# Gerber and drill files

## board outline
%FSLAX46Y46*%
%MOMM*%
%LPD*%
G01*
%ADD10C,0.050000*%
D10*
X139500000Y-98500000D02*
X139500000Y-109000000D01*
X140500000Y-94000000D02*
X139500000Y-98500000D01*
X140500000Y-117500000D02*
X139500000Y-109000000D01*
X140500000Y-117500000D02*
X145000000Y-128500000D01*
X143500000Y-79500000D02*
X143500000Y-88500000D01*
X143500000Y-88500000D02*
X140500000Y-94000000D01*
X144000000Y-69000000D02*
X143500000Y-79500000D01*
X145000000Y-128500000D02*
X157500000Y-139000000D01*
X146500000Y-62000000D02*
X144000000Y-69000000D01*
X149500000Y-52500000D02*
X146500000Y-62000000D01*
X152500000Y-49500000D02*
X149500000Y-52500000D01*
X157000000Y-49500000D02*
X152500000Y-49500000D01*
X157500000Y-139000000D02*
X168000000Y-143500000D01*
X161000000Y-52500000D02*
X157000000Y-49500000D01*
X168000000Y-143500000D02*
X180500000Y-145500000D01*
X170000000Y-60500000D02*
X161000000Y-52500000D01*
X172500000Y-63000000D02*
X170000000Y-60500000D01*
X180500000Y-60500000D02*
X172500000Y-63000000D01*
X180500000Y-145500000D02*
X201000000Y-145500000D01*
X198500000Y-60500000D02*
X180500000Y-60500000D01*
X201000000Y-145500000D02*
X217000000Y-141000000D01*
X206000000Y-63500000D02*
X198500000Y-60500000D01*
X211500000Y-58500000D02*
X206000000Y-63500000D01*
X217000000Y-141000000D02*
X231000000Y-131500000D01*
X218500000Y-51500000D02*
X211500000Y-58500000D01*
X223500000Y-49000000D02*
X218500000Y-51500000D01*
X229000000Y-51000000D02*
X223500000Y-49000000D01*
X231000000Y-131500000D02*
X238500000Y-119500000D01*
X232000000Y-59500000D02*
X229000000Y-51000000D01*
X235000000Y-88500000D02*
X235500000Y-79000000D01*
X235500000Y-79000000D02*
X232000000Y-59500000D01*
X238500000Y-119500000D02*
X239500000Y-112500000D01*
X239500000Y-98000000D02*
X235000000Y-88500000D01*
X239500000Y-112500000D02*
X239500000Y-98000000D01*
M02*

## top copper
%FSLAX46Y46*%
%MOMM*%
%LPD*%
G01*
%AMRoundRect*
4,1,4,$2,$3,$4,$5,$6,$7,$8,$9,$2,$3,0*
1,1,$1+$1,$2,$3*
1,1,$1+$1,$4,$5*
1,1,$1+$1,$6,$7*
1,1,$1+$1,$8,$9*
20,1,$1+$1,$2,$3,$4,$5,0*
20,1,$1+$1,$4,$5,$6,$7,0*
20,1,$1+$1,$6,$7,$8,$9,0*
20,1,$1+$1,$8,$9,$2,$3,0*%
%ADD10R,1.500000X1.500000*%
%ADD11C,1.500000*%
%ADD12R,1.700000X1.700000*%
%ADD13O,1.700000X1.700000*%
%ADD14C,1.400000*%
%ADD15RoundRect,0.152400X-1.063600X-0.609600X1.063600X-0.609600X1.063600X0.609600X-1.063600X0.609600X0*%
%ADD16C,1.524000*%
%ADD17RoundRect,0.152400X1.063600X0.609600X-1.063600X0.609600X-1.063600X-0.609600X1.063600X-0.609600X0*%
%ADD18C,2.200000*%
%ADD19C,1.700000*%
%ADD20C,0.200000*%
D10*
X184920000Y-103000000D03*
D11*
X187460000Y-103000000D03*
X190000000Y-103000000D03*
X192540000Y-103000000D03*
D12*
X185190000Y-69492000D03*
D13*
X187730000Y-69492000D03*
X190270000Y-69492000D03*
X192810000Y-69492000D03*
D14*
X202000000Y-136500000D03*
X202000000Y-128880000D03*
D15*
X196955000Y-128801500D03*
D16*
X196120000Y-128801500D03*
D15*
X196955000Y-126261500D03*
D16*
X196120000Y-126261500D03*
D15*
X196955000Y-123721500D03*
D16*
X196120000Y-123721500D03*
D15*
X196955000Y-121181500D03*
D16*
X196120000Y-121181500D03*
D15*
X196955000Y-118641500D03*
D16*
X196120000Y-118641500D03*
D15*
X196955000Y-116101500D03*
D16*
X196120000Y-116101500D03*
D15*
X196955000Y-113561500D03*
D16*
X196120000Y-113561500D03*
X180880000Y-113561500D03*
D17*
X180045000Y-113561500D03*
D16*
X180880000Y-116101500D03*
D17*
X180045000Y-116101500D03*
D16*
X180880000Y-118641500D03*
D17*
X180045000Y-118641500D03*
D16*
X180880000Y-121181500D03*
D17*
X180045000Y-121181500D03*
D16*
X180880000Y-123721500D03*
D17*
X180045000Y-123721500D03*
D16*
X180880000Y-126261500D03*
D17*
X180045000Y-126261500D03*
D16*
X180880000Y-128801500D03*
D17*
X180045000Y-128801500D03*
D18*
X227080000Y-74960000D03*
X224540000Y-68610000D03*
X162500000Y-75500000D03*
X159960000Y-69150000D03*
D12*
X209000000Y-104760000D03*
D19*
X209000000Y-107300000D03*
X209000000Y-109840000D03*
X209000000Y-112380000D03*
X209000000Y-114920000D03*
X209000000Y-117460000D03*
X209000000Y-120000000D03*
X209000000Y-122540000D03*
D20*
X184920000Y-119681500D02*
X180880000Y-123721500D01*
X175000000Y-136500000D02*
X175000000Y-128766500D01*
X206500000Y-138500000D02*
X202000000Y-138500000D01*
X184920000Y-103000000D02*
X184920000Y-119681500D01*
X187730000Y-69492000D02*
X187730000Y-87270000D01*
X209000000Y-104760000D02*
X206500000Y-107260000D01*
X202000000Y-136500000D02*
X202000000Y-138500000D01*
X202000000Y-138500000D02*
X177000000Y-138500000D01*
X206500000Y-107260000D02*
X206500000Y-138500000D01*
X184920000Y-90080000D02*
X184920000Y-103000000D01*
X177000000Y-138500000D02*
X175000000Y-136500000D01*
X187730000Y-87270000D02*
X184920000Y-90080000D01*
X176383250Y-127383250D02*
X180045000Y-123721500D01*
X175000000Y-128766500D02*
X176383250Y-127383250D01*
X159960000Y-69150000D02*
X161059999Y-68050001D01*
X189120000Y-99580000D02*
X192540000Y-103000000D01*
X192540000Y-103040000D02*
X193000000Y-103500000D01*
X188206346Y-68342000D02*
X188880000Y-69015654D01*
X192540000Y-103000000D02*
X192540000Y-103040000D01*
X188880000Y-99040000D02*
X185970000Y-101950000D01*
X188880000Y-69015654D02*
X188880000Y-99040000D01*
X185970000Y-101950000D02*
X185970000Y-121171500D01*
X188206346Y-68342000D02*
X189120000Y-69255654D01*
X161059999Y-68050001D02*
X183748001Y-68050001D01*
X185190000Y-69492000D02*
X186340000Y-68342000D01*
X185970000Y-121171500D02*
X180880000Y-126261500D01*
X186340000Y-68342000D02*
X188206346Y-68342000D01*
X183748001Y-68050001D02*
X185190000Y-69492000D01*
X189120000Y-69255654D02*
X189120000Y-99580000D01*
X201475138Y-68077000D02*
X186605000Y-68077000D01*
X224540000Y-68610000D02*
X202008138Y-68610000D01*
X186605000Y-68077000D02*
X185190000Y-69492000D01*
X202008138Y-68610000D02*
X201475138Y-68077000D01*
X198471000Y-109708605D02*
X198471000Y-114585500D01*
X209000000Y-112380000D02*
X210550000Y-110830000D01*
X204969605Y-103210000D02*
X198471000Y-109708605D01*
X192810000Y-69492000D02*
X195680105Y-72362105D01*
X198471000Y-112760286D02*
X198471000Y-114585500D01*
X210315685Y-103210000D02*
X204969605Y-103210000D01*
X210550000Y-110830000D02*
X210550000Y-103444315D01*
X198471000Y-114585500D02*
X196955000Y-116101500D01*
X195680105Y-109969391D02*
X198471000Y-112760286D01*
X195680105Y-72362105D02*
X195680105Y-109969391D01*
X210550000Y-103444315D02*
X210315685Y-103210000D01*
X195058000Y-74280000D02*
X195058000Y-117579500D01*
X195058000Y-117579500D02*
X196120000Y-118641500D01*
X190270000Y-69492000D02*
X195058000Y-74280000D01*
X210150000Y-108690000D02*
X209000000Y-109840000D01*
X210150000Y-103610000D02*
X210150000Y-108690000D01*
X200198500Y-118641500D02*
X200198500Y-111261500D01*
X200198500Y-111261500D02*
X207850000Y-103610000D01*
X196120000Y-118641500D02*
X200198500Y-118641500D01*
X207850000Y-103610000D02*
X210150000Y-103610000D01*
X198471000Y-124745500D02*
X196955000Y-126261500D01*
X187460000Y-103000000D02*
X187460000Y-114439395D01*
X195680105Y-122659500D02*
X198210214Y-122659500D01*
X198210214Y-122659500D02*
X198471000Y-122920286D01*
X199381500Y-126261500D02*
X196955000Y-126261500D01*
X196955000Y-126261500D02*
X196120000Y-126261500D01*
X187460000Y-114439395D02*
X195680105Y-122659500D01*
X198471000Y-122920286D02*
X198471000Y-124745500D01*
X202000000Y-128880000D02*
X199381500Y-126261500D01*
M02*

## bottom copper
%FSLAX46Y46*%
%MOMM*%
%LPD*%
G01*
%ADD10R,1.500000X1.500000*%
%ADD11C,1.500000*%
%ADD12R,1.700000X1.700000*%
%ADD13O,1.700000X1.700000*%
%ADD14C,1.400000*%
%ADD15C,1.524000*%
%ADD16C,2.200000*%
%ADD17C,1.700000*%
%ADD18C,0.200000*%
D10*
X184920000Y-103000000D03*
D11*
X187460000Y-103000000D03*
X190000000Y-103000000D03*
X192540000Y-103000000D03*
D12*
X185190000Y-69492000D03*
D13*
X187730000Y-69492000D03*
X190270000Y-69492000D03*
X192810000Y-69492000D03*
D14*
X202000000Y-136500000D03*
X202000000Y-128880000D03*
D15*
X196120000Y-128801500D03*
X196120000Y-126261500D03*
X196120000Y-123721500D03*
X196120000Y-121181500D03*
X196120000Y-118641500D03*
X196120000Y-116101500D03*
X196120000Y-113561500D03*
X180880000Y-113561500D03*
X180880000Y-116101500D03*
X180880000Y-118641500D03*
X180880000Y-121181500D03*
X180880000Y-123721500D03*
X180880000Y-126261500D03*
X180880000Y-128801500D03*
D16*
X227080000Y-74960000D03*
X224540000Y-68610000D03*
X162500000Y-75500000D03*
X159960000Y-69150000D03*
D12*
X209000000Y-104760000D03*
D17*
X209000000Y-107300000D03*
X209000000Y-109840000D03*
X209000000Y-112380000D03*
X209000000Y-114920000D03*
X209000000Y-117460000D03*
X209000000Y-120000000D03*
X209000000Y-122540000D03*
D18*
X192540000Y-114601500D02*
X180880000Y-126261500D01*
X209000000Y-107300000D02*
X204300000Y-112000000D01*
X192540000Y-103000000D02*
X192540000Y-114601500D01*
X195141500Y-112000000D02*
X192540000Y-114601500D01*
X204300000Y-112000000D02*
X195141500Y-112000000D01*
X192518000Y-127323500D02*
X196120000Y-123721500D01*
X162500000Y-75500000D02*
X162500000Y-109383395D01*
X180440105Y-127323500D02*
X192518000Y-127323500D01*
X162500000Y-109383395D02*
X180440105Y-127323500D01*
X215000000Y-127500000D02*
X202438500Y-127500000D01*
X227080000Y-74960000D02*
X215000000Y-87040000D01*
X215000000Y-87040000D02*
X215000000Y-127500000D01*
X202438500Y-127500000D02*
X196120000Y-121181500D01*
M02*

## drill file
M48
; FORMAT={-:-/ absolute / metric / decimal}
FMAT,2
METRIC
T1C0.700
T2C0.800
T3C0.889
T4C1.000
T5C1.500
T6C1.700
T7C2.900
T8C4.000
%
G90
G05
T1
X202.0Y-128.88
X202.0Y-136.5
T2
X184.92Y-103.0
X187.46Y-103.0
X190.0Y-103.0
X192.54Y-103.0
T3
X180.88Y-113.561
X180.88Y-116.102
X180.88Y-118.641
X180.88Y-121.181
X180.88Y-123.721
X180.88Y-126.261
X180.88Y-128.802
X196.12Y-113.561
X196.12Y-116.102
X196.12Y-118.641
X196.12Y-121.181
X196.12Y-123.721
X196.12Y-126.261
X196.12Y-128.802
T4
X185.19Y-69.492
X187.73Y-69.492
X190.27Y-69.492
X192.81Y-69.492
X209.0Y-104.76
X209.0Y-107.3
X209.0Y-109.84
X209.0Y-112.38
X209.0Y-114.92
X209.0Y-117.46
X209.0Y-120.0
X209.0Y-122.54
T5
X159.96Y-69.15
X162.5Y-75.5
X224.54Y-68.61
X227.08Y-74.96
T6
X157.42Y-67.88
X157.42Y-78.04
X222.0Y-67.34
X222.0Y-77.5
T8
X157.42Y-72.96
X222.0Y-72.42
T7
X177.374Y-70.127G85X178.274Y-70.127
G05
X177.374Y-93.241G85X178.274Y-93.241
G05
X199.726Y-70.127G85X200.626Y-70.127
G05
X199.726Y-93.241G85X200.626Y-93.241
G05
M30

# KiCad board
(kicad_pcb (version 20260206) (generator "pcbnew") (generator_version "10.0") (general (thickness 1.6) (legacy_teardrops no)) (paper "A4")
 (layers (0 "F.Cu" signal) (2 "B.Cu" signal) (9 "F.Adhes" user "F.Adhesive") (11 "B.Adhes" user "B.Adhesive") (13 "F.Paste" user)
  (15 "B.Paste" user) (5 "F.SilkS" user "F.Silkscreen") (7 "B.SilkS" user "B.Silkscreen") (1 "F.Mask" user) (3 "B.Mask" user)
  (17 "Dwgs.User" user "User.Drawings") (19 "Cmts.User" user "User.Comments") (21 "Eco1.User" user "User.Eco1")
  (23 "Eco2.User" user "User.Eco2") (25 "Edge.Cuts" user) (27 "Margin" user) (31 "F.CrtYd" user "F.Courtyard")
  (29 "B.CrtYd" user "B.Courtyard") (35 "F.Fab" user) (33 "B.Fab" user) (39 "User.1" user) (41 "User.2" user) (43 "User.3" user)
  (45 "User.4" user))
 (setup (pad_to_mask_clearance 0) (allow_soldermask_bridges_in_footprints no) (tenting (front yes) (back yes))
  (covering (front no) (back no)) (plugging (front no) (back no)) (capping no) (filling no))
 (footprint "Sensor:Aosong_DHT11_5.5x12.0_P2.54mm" (layer "F.Cu") (at 184.92 103 90)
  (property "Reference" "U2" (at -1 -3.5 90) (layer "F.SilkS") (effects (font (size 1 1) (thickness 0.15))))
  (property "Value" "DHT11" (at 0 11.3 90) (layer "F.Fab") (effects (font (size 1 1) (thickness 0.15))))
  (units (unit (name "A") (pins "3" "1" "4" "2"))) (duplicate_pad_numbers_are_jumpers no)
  (pad "1" thru_hole rect (at 0 0 90) (size 1.5 1.5) (drill 0.8) (layers "*.Cu" "*.Mask") (remove_unused_layers no) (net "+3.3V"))
  (pad "2" thru_hole circle (at 0 2.54 90) (size 1.5 1.5) (drill 0.8) (layers "*.Cu" "*.Mask") (remove_unused_layers no) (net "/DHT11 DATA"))
  (pad "3" thru_hole circle (at 0 5.08 90) (size 1.5 1.5) (drill 0.8) (layers "*.Cu" "*.Mask") (remove_unused_layers no)
   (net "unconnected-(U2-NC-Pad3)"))
  (pad "4" thru_hole circle (at 0 7.62 90) (size 1.5 1.5) (drill 0.8) (layers "*.Cu" "*.Mask") (remove_unused_layers no) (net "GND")))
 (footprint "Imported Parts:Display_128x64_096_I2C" (layer "F.Cu") (at 189 69.492)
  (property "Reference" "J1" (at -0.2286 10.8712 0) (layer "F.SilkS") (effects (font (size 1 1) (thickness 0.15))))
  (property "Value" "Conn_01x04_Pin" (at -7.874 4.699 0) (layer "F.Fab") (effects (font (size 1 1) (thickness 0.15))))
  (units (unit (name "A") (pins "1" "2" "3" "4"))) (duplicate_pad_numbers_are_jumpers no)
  (pad "" np_thru_hole oval (at -11.176 0.635) (size 3.8 2.9) (drill oval 3.8 2.9) (layers "*.Cu" "*.Mask"))
  (pad "" np_thru_hole oval (at -11.176 23.749) (size 3.8 2.9) (drill oval 3.8 2.9) (layers "*.Cu" "*.Mask"))
  (pad "" np_thru_hole oval (at 11.176 0.635) (size 3.8 2.9) (drill oval 3.8 2.9) (layers "*.Cu" "*.Mask"))
  (pad "" np_thru_hole oval (at 11.176 23.749) (size 3.8 2.9) (drill oval 3.8 2.9) (layers "*.Cu" "*.Mask"))
  (pad "1" thru_hole rect (at -3.81 0 90) (size 1.7 1.7) (drill 1) (layers "*.Cu" "*.Mask") (remove_unused_layers no) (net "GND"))
  (pad "2" thru_hole oval (at -1.27 0 90) (size 1.7 1.7) (drill 1) (layers "*.Cu" "*.Mask") (remove_unused_layers no) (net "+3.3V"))
  (pad "3" thru_hole oval (at 1.27 0 90) (size 1.7 1.7) (drill 1) (layers "*.Cu" "*.Mask") (remove_unused_layers no) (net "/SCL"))
  (pad "4" thru_hole oval (at 3.81 0 90) (size 1.7 1.7) (drill 1) (layers "*.Cu" "*.Mask") (remove_unused_layers no) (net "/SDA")))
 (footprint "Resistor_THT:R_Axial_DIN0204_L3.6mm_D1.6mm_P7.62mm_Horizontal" (layer "F.Cu") (at 202 136.5 90)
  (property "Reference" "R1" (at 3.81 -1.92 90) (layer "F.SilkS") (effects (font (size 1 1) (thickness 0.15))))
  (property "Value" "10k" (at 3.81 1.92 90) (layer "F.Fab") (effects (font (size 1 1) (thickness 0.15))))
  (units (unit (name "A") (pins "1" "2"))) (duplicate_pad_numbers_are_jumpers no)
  (pad "1" thru_hole circle (at 0 0 90) (size 1.4 1.4) (drill 0.7) (layers "*.Cu" "*.Mask") (remove_unused_layers no) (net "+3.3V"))
  (pad "2" thru_hole circle (at 7.62 0 90) (size 1.4 1.4) (drill 0.7) (layers "*.Cu" "*.Mask") (remove_unused_layers no) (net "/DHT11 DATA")))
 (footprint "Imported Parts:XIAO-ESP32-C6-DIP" (layer "F.Cu") (at 188.5 121.1815 -90)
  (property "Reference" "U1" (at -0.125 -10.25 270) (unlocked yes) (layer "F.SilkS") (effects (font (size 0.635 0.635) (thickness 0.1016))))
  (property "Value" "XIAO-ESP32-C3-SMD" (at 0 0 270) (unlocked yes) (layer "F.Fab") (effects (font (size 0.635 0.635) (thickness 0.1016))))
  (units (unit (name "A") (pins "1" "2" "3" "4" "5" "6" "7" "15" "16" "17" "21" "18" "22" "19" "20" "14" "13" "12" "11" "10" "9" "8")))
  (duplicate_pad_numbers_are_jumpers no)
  (pad "1" smd roundrect (at 7.62 -8.455) (size 2.432 1.524) (layers "F.Cu" "F.Mask") (roundrect_rratio 0.1)
   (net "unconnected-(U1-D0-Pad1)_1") (thermal_bridge_angle 45))
  (pad "1" thru_hole circle (at 7.62 -7.62) (size 1.524 1.524) (drill 0.889) (layers "*.Cu" "*.Mask") (remove_unused_layers no)
   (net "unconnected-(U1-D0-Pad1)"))
  (pad "2" smd roundrect (at 5.08 -8.455) (size 2.432 1.524) (layers "F.Cu" "F.Mask") (roundrect_rratio 0.1) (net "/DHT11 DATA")
   (thermal_bridge_angle 45))
  (pad "2" thru_hole circle (at 5.08 -7.62) (size 1.524 1.524) (drill 0.889) (layers "*.Cu" "*.Mask") (remove_unused_layers no)
   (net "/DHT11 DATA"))
  (pad "3" smd roundrect (at 2.54 -8.455) (size 2.432 1.524) (layers "F.Cu" "F.Mask") (roundrect_rratio 0.1) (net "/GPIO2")
   (thermal_bridge_angle 45))
  (pad "3" thru_hole circle (at 2.54 -7.62) (size 1.524 1.524) (drill 0.889) (layers "*.Cu" "*.Mask") (remove_unused_layers no)
   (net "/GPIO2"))
  (pad "4" smd roundrect (at 0 -8.455) (size 2.432 1.524) (layers "F.Cu" "F.Mask") (roundrect_rratio 0.1) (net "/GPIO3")
   (thermal_bridge_angle 45))
  (pad "4" thru_hole circle (at 0 -7.62) (size 1.524 1.524) (drill 0.889) (layers "*.Cu" "*.Mask") (remove_unused_layers no) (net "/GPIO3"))
  (pad "5" smd roundrect (at -2.54 -8.455) (size 2.432 1.524) (layers "F.Cu" "F.Mask") (roundrect_rratio 0.1) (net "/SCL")
   (thermal_bridge_angle 45))
  (pad "5" thru_hole circle (at -2.54 -7.62) (size 1.524 1.524) (drill 0.889) (layers "*.Cu" "*.Mask") (remove_unused_layers no)
   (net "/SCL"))
  (pad "6" smd roundrect (at -5.08 -8.455) (size 2.432 1.524) (layers "F.Cu" "F.Mask") (roundrect_rratio 0.1) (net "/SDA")
   (thermal_bridge_angle 45))
  (pad "6" thru_hole circle (at -5.08 -7.62) (size 1.524 1.524) (drill 0.889) (layers "*.Cu" "*.Mask") (remove_unused_layers no)
   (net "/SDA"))
  (pad "7" smd roundrect (at -7.62 -8.455) (size 2.432 1.524) (layers "F.Cu" "F.Mask") (roundrect_rratio 0.1)
   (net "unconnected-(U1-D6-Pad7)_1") (thermal_bridge_angle 45))
  (pad "7" thru_hole circle (at -7.62 -7.62) (size 1.524 1.524) (drill 0.889) (layers "*.Cu" "*.Mask") (remove_unused_layers no)
   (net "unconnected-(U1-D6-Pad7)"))
  (pad "8" thru_hole circle (at -7.62 7.62 180) (size 1.524 1.524) (drill 0.889) (layers "*.Cu" "*.Mask") (remove_unused_layers no)
   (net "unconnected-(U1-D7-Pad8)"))
  (pad "8" smd roundrect (at -7.62 8.455 180) (size 2.432 1.524) (layers "F.Cu" "F.Mask") (roundrect_rratio 0.1)
   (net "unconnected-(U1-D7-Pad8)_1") (thermal_bridge_angle 45))
  (pad "9" thru_hole circle (at -5.08 7.62 180) (size 1.524 1.524) (drill 0.889) (layers "*.Cu" "*.Mask") (remove_unused_layers no)
   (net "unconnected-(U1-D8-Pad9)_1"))
  (pad "9" smd roundrect (at -5.08 8.455 180) (size 2.432 1.524) (layers "F.Cu" "F.Mask") (roundrect_rratio 0.1)
   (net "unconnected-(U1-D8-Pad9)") (thermal_bridge_angle 45))
  (pad "10" thru_hole circle (at -2.54 7.62 180) (size 1.524 1.524) (drill 0.889) (layers "*.Cu" "*.Mask") (remove_unused_layers no)
   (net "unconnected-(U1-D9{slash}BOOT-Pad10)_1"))
  (pad "10" smd roundrect (at -2.54 8.455 180) (size 2.432 1.524) (layers "F.Cu" "F.Mask") (roundrect_rratio 0.1)
   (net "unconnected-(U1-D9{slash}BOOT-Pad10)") (thermal_bridge_angle 45))
  (pad "11" thru_hole circle (at 0 7.62 180) (size 1.524 1.524) (drill 0.889) (layers "*.Cu" "*.Mask") (remove_unused_layers no)
   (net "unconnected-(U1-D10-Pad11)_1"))
  (pad "11" smd roundrect (at 0 8.455 180) (size 2.432 1.524) (layers "F.Cu" "F.Mask") (roundrect_rratio 0.1)
   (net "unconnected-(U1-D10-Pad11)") (thermal_bridge_angle 45))
  (pad "12" thru_hole circle (at 2.54 7.62 180) (size 1.524 1.524) (drill 0.889) (layers "*.Cu" "*.Mask") (remove_unused_layers no)
   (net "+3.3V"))
  (pad "12" smd roundrect (at 2.54 8.455 180) (size 2.432 1.524) (layers "F.Cu" "F.Mask") (roundrect_rratio 0.1) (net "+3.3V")
   (thermal_bridge_angle 45))
  (pad "13" thru_hole circle (at 5.08 7.62 180) (size 1.524 1.524) (drill 0.889) (layers "*.Cu" "*.Mask") (remove_unused_layers no)
   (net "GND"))
  (pad "13" smd roundrect (at 5.08 8.455 180) (size 2.432 1.524) (layers "F.Cu" "F.Mask") (roundrect_rratio 0.1) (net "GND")
   (thermal_bridge_angle 45))
  (pad "14" thru_hole circle (at 7.62 7.62 180) (size 1.524 1.524) (drill 0.889) (layers "*.Cu" "*.Mask") (remove_unused_layers no)
   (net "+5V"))
  (pad "14" smd roundrect (at 7.62 8.455 180) (size 2.432 1.524) (layers "F.Cu" "F.Mask") (roundrect_rratio 0.1) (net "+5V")
   (thermal_bridge_angle 45)))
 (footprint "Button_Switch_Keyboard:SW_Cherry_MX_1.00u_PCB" (layer "F.Cu") (at 227.08 74.96 -90)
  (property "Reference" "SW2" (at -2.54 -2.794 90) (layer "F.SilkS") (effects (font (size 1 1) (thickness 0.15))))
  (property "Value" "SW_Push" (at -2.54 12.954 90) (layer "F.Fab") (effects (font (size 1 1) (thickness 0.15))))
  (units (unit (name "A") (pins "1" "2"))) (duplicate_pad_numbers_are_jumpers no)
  (pad "" np_thru_hole circle (at -7.62 5.08 270) (size 1.7 1.7) (drill 1.7) (layers "*.Cu" "*.Mask"))
  (pad "" np_thru_hole circle (at -2.54 5.08 270) (size 4 4) (drill 4) (layers "*.Cu" "*.Mask"))
  (pad "" np_thru_hole circle (at 2.54 5.08 270) (size 1.7 1.7) (drill 1.7) (layers "*.Cu" "*.Mask"))
  (pad "1" thru_hole circle (at 0 0 270) (size 2.2 2.2) (drill 1.5) (layers "*.Cu" "*.Mask") (remove_unused_layers no) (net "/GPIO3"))
  (pad "2" thru_hole circle (at -6.35 2.54 270) (size 2.2 2.2) (drill 1.5) (layers "*.Cu" "*.Mask") (remove_unused_layers no) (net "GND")))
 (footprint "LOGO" (layer "F.Cu") (at 161 108.5)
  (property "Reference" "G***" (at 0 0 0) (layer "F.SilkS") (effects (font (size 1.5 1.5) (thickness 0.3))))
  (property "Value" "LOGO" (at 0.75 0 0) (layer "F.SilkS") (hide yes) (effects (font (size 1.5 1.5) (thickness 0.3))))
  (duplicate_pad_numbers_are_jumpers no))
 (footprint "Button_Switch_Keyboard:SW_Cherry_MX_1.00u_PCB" (layer "F.Cu") (at 162.5 75.5 -90)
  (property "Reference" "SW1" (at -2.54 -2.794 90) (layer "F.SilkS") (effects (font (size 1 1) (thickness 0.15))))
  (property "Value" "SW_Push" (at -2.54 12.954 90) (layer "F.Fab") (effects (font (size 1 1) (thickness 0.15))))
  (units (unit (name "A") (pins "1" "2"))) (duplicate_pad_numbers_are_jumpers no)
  (pad "" np_thru_hole circle (at -7.62 5.08 270) (size 1.7 1.7) (drill 1.7) (layers "*.Cu" "*.Mask"))
  (pad "" np_thru_hole circle (at -2.54 5.08 270) (size 4 4) (drill 4) (layers "*.Cu" "*.Mask"))
  (pad "" np_thru_hole circle (at 2.54 5.08 270) (size 1.7 1.7) (drill 1.7) (layers "*.Cu" "*.Mask"))
  (pad "1" thru_hole circle (at 0 0 270) (size 2.2 2.2) (drill 1.5) (layers "*.Cu" "*.Mask") (remove_unused_layers no) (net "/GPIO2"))
  (pad "2" thru_hole circle (at -6.35 2.54 270) (size 2.2 2.2) (drill 1.5) (layers "*.Cu" "*.Mask") (remove_unused_layers no) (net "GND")))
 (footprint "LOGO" (layer "F.Cu") (at 221.5 91)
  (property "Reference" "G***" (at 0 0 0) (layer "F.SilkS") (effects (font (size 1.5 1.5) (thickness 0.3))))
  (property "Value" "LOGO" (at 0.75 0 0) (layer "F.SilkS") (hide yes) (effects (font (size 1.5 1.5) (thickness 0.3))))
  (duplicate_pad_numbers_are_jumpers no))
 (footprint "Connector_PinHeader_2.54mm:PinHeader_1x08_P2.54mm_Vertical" (layer "F.Cu") (at 209 104.76)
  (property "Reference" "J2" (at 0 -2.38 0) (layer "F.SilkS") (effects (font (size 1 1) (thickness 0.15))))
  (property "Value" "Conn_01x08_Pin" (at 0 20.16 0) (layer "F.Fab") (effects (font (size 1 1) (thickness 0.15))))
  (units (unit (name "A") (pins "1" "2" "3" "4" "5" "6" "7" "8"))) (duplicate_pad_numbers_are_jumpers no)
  (pad "1" thru_hole rect (at 0 0) (size 1.7 1.7) (drill 1) (layers "*.Cu" "*.Mask") (remove_unused_layers no) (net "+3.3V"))
  (pad "2" thru_hole circle (at 0 2.54) (size 1.7 1.7) (drill 1) (layers "*.Cu" "*.Mask") (remove_unused_layers no) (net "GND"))
  (pad "3" thru_hole circle (at 0 5.08) (size 1.7 1.7) (drill 1) (layers "*.Cu" "*.Mask") (remove_unused_layers no) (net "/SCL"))
  (pad "4" thru_hole circle (at 0 7.62) (size 1.7 1.7) (drill 1) (layers "*.Cu" "*.Mask") (remove_unused_layers no) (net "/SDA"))
  (pad "5" thru_hole circle (at 0 10.16) (size 1.7 1.7) (drill 1) (layers "*.Cu" "*.Mask") (remove_unused_layers no)
   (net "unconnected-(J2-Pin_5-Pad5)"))
  (pad "6" thru_hole circle (at 0 12.7) (size 1.7 1.7) (drill 1) (layers "*.Cu" "*.Mask") (remove_unused_layers no)
   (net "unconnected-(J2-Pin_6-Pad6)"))
  (pad "7" thru_hole circle (at 0 15.24) (size 1.7 1.7) (drill 1) (layers "*.Cu" "*.Mask") (remove_unused_layers no)
   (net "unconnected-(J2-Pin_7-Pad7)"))
  (pad "8" thru_hole circle (at 0 17.78) (size 1.7 1.7) (drill 1) (layers "*.Cu" "*.Mask") (remove_unused_layers no)
   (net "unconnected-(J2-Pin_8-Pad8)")))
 (gr_line (start 139.5 98.5) (end 139.5 109) (stroke (width 0.05) (type default)) (layer "Edge.Cuts"))
 (gr_line (start 140.5 94) (end 139.5 98.5) (stroke (width 0.05) (type default)) (layer "Edge.Cuts"))
 (gr_line (start 140.5 117.5) (end 139.5 109) (stroke (width 0.05) (type default)) (layer "Edge.Cuts"))
 (gr_line (start 140.5 117.5) (end 145 128.5) (stroke (width 0.05) (type default)) (layer "Edge.Cuts"))
 (gr_line (start 143.5 79.5) (end 143.5 88.5) (stroke (width 0.05) (type default)) (layer "Edge.Cuts"))
 (gr_line (start 143.5 88.5) (end 140.5 94) (stroke (width 0.05) (type default)) (layer "Edge.Cuts"))
 (gr_line (start 144 69) (end 143.5 79.5) (stroke (width 0.05) (type default)) (layer "Edge.Cuts"))
 (gr_line (start 145 128.5) (end 157.5 139) (stroke (width 0.05) (type default)) (layer "Edge.Cuts"))
 (gr_line (start 146.5 62) (end 144 69) (stroke (width 0.05) (type default)) (layer "Edge.Cuts"))
 (gr_line (start 149.5 52.5) (end 146.5 62) (stroke (width 0.05) (type default)) (layer "Edge.Cuts"))
 (gr_line (start 152.5 49.5) (end 149.5 52.5) (stroke (width 0.05) (type default)) (layer "Edge.Cuts"))
 (gr_line (start 157 49.5) (end 152.5 49.5) (stroke (width 0.05) (type default)) (layer "Edge.Cuts"))
 (gr_line (start 157.5 139) (end 168 143.5) (stroke (width 0.05) (type default)) (layer "Edge.Cuts"))
 (gr_line (start 161 52.5) (end 157 49.5) (stroke (width 0.05) (type default)) (layer "Edge.Cuts"))
 (gr_line (start 168 143.5) (end 180.5 145.5) (stroke (width 0.05) (type default)) (layer "Edge.Cuts"))
 (gr_line (start 170 60.5) (end 161 52.5) (stroke (width 0.05) (type default)) (layer "Edge.Cuts"))
 (gr_line (start 172.5 63) (end 170 60.5) (stroke (width 0.05) (type default)) (layer "Edge.Cuts"))
 (gr_line (start 180.5 60.5) (end 172.5 63) (stroke (width 0.05) (type default)) (layer "Edge.Cuts"))
 (gr_line (start 180.5 145.5) (end 201 145.5) (stroke (width 0.05) (type default)) (layer "Edge.Cuts"))
 (gr_line (start 198.5 60.5) (end 180.5 60.5) (stroke (width 0.05) (type default)) (layer "Edge.Cuts"))
 (gr_line (start 201 145.5) (end 217 141) (stroke (width 0.05) (type default)) (layer "Edge.Cuts"))
 (gr_line (start 206 63.5) (end 198.5 60.5) (stroke (width 0.05) (type default)) (layer "Edge.Cuts"))
 (gr_line (start 211.5 58.5) (end 206 63.5) (stroke (width 0.05) (type default)) (layer "Edge.Cuts"))
 (gr_line (start 217 141) (end 231 131.5) (stroke (width 0.05) (type default)) (layer "Edge.Cuts"))
 (gr_line (start 218.5 51.5) (end 211.5 58.5) (stroke (width 0.05) (type default)) (layer "Edge.Cuts"))
 (gr_line (start 223.5 49) (end 218.5 51.5) (stroke (width 0.05) (type default)) (layer "Edge.Cuts"))
 (gr_line (start 229 51) (end 223.5 49) (stroke (width 0.05) (type default)) (layer "Edge.Cuts"))
 (gr_line (start 231 131.5) (end 238.5 119.5) (stroke (width 0.05) (type default)) (layer "Edge.Cuts"))
 (gr_line (start 232 59.5) (end 229 51) (stroke (width 0.05) (type default)) (layer "Edge.Cuts"))
 (gr_line (start 235 88.5) (end 235.5 79) (stroke (width 0.05) (type default)) (layer "Edge.Cuts"))
 (gr_line (start 235.5 79) (end 232 59.5) (stroke (width 0.05) (type default)) (layer "Edge.Cuts"))
 (gr_line (start 238.5 119.5) (end 239.5 112.5) (stroke (width 0.05) (type default)) (layer "Edge.Cuts"))
 (gr_line (start 239.5 98) (end 235 88.5) (stroke (width 0.05) (type default)) (layer "Edge.Cuts"))
 (gr_line (start 239.5 112.5) (end 239.5 98) (stroke (width 0.05) (type default)) (layer "Edge.Cuts"))
 (segment (start 184.92 119.6815) (end 180.88 123.7215) (width 0.2) (layer "F.Cu") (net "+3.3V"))
 (segment (start 175 136.5) (end 175 128.7665) (width 0.2) (layer "F.Cu") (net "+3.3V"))
 (segment (start 206.5 138.5) (end 202 138.5) (width 0.2) (layer "F.Cu") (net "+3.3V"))
 (segment (start 184.92 103) (end 184.92 119.6815) (width 0.2) (layer "F.Cu") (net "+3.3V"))
 (segment (start 187.73 69.492) (end 187.73 87.27) (width 0.2) (layer "F.Cu") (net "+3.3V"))
 (segment (start 209 104.76) (end 206.5 107.26) (width 0.2) (layer "F.Cu") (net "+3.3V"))
 (segment (start 202 136.5) (end 202 138.5) (width 0.2) (layer "F.Cu") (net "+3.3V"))
 (segment (start 202 138.5) (end 177 138.5) (width 0.2) (layer "F.Cu") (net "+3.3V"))
 (segment (start 206.5 107.26) (end 206.5 138.5) (width 0.2) (layer "F.Cu") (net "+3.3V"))
 (segment (start 184.92 90.08) (end 184.92 103) (width 0.2) (layer "F.Cu") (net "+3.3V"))
 (segment (start 177 138.5) (end 175 136.5) (width 0.2) (layer "F.Cu") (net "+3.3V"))
 (segment (start 187.73 87.27) (end 184.92 90.08) (width 0.2) (layer "F.Cu") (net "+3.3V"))
 (segment (start 176.38325 127.38325) (end 180.045 123.7215) (width 0.2) (layer "F.Cu") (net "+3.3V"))
 (segment (start 175 128.7665) (end 176.38325 127.38325) (width 0.2) (layer "F.Cu") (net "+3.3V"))
 (segment (start 159.96 69.15) (end 161.059999 68.050001) (width 0.2) (layer "F.Cu") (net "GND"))
 (segment (start 189.12 99.58) (end 192.54 103) (width 0.2) (layer "F.Cu") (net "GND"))
 (segment (start 192.54 103.04) (end 193 103.5) (width 0.2) (layer "F.Cu") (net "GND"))
 (segment (start 188.206346 68.342) (end 188.88 69.015654) (width 0.2) (layer "F.Cu") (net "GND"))
 (segment (start 192.54 103) (end 192.54 103.04) (width 0.2) (layer "F.Cu") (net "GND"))
 (segment (start 188.88 99.04) (end 185.97 101.95) (width 0.2) (layer "F.Cu") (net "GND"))
 (segment (start 188.88 69.015654) (end 188.88 99.04) (width 0.2) (layer "F.Cu") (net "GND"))
 (segment (start 185.97 101.95) (end 185.97 121.1715) (width 0.2) (layer "F.Cu") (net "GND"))
 (segment (start 188.206346 68.342) (end 189.12 69.255654) (width 0.2) (layer "F.Cu") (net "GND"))
 (segment (start 161.059999 68.050001) (end 183.748001 68.050001) (width 0.2) (layer "F.Cu") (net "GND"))
 (segment (start 185.19 69.492) (end 186.34 68.342) (width 0.2) (layer "F.Cu") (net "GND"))
 (segment (start 185.97 121.1715) (end 180.88 126.2615) (width 0.2) (layer "F.Cu") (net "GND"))
 (segment (start 186.34 68.342) (end 188.206346 68.342) (width 0.2) (layer "F.Cu") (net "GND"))
 (segment (start 183.748001 68.050001) (end 185.19 69.492) (width 0.2) (layer "F.Cu") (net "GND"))
 (segment (start 189.12 69.255654) (end 189.12 99.58) (width 0.2) (layer "F.Cu") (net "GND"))
 (segment (start 201.475138 68.077) (end 186.605 68.077) (width 0.2) (layer "F.Cu") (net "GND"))
 (segment (start 224.54 68.61) (end 202.008138 68.61) (width 0.2) (layer "F.Cu") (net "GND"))
 (segment (start 186.605 68.077) (end 185.19 69.492) (width 0.2) (layer "F.Cu") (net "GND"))
 (segment (start 202.008138 68.61) (end 201.475138 68.077) (width 0.2) (layer "F.Cu") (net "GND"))
 (segment (start 192.54 114.6015) (end 180.88 126.2615) (width 0.2) (layer "B.Cu") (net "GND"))
 (segment (start 209 107.3) (end 204.3 112) (width 0.2) (layer "B.Cu") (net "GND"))
 (segment (start 192.54 103) (end 192.54 114.6015) (width 0.2) (layer "B.Cu") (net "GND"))
 (segment (start 195.1415 112) (end 192.54 114.6015) (width 0.2) (layer "B.Cu") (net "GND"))
 (segment (start 204.3 112) (end 195.1415 112) (width 0.2) (layer "B.Cu") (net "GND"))
 (segment (start 198.471 109.708605) (end 198.471 114.5855) (width 0.2) (layer "F.Cu") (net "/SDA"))
 (segment (start 209 112.38) (end 210.55 110.83) (width 0.2) (layer "F.Cu") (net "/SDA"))
 (segment (start 204.969605 103.21) (end 198.471 109.708605) (width 0.2) (layer "F.Cu") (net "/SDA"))
 (segment (start 192.81 69.492) (end 195.680105 72.362105) (width 0.2) (layer "F.Cu") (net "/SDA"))
 (segment (start 198.471 112.760286) (end 198.471 114.5855) (width 0.2) (layer "F.Cu") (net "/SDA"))
 (segment (start 210.315685 103.21) (end 204.969605 103.21) (width 0.2) (layer "F.Cu") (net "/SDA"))
 (segment (start 210.55 110.83) (end 210.55 103.444315) (width 0.2) (layer "F.Cu") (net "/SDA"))
 (segment (start 198.471 114.5855) (end 196.955 116.1015) (width 0.2) (layer "F.Cu") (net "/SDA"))
 (segment (start 195.680105 109.969391) (end 198.471 112.760286) (width 0.2) (layer "F.Cu") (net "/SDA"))
 (segment (start 195.680105 72.362105) (end 195.680105 109.969391) (width 0.2) (layer "F.Cu") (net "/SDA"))
 (segment (start 210.55 103.444315) (end 210.315685 103.21) (width 0.2) (layer "F.Cu") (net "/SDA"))
 (segment (start 195.058 74.28) (end 195.058 117.5795) (width 0.2) (layer "F.Cu") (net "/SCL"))
 (segment (start 195.058 117.5795) (end 196.12 118.6415) (width 0.2) (layer "F.Cu") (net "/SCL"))
 (segment (start 190.27 69.492) (end 195.058 74.28) (width 0.2) (layer "F.Cu") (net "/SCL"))
 (segment (start 210.15 108.69) (end 209 109.84) (width 0.2) (layer "F.Cu") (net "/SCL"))
 (segment (start 210.15 103.61) (end 210.15 108.69) (width 0.2) (layer "F.Cu") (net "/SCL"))
 (segment (start 200.1985 118.6415) (end 200.1985 111.2615) (width 0.2) (layer "F.Cu") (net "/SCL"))
 (segment (start 200.1985 111.2615) (end 207.85 103.61) (width 0.2) (layer "F.Cu") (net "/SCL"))
 (segment (start 196.12 118.6415) (end 200.1985 118.6415) (width 0.2) (layer "F.Cu") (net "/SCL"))
 (segment (start 207.85 103.61) (end 210.15 103.61) (width 0.2) (layer "F.Cu") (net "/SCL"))
 (segment (start 198.471 124.7455) (end 196.955 126.2615) (width 0.2) (layer "F.Cu") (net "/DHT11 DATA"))
 (segment (start 187.46 103) (end 187.46 114.439395) (width 0.2) (layer "F.Cu") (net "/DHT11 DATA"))
 (segment (start 195.680105 122.6595) (end 198.210214 122.6595) (width 0.2) (layer "F.Cu") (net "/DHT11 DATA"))
 (segment (start 198.210214 122.6595) (end 198.471 122.920286) (width 0.2) (layer "F.Cu") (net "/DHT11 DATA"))
 (segment (start 199.3815 126.2615) (end 196.955 126.2615) (width 0.2) (layer "F.Cu") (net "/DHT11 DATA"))
 (segment (start 196.955 126.2615) (end 196.12 126.2615) (width 0.2) (layer "F.Cu") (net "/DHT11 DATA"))
 (segment (start 187.46 114.439395) (end 195.680105 122.6595) (width 0.2) (layer "F.Cu") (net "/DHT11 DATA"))
 (segment (start 198.471 122.920286) (end 198.471 124.7455) (width 0.2) (layer "F.Cu") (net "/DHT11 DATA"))
 (segment (start 202 128.88) (end 199.3815 126.2615) (width 0.2) (layer "F.Cu") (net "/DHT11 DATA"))
 (segment (start 192.518 127.3235) (end 196.12 123.7215) (width 0.2) (layer "B.Cu") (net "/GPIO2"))
 (segment (start 162.5 75.5) (end 162.5 109.383395) (width 0.2) (layer "B.Cu") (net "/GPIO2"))
 (segment (start 180.440105 127.3235) (end 192.518 127.3235) (width 0.2) (layer "B.Cu") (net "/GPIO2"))
 (segment (start 162.5 109.383395) (end 180.440105 127.3235) (width 0.2) (layer "B.Cu") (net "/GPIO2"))
 (segment (start 215 127.5) (end 202.4385 127.5) (width 0.2) (layer "B.Cu") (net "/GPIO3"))
 (segment (start 227.08 74.96) (end 215 87.04) (width 0.2) (layer "B.Cu") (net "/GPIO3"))
 (segment (start 215 87.04) (end 215 127.5) (width 0.2) (layer "B.Cu") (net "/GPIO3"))
 (segment (start 202.4385 127.5) (end 196.12 121.1815) (width 0.2) (layer "B.Cu") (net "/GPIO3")))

